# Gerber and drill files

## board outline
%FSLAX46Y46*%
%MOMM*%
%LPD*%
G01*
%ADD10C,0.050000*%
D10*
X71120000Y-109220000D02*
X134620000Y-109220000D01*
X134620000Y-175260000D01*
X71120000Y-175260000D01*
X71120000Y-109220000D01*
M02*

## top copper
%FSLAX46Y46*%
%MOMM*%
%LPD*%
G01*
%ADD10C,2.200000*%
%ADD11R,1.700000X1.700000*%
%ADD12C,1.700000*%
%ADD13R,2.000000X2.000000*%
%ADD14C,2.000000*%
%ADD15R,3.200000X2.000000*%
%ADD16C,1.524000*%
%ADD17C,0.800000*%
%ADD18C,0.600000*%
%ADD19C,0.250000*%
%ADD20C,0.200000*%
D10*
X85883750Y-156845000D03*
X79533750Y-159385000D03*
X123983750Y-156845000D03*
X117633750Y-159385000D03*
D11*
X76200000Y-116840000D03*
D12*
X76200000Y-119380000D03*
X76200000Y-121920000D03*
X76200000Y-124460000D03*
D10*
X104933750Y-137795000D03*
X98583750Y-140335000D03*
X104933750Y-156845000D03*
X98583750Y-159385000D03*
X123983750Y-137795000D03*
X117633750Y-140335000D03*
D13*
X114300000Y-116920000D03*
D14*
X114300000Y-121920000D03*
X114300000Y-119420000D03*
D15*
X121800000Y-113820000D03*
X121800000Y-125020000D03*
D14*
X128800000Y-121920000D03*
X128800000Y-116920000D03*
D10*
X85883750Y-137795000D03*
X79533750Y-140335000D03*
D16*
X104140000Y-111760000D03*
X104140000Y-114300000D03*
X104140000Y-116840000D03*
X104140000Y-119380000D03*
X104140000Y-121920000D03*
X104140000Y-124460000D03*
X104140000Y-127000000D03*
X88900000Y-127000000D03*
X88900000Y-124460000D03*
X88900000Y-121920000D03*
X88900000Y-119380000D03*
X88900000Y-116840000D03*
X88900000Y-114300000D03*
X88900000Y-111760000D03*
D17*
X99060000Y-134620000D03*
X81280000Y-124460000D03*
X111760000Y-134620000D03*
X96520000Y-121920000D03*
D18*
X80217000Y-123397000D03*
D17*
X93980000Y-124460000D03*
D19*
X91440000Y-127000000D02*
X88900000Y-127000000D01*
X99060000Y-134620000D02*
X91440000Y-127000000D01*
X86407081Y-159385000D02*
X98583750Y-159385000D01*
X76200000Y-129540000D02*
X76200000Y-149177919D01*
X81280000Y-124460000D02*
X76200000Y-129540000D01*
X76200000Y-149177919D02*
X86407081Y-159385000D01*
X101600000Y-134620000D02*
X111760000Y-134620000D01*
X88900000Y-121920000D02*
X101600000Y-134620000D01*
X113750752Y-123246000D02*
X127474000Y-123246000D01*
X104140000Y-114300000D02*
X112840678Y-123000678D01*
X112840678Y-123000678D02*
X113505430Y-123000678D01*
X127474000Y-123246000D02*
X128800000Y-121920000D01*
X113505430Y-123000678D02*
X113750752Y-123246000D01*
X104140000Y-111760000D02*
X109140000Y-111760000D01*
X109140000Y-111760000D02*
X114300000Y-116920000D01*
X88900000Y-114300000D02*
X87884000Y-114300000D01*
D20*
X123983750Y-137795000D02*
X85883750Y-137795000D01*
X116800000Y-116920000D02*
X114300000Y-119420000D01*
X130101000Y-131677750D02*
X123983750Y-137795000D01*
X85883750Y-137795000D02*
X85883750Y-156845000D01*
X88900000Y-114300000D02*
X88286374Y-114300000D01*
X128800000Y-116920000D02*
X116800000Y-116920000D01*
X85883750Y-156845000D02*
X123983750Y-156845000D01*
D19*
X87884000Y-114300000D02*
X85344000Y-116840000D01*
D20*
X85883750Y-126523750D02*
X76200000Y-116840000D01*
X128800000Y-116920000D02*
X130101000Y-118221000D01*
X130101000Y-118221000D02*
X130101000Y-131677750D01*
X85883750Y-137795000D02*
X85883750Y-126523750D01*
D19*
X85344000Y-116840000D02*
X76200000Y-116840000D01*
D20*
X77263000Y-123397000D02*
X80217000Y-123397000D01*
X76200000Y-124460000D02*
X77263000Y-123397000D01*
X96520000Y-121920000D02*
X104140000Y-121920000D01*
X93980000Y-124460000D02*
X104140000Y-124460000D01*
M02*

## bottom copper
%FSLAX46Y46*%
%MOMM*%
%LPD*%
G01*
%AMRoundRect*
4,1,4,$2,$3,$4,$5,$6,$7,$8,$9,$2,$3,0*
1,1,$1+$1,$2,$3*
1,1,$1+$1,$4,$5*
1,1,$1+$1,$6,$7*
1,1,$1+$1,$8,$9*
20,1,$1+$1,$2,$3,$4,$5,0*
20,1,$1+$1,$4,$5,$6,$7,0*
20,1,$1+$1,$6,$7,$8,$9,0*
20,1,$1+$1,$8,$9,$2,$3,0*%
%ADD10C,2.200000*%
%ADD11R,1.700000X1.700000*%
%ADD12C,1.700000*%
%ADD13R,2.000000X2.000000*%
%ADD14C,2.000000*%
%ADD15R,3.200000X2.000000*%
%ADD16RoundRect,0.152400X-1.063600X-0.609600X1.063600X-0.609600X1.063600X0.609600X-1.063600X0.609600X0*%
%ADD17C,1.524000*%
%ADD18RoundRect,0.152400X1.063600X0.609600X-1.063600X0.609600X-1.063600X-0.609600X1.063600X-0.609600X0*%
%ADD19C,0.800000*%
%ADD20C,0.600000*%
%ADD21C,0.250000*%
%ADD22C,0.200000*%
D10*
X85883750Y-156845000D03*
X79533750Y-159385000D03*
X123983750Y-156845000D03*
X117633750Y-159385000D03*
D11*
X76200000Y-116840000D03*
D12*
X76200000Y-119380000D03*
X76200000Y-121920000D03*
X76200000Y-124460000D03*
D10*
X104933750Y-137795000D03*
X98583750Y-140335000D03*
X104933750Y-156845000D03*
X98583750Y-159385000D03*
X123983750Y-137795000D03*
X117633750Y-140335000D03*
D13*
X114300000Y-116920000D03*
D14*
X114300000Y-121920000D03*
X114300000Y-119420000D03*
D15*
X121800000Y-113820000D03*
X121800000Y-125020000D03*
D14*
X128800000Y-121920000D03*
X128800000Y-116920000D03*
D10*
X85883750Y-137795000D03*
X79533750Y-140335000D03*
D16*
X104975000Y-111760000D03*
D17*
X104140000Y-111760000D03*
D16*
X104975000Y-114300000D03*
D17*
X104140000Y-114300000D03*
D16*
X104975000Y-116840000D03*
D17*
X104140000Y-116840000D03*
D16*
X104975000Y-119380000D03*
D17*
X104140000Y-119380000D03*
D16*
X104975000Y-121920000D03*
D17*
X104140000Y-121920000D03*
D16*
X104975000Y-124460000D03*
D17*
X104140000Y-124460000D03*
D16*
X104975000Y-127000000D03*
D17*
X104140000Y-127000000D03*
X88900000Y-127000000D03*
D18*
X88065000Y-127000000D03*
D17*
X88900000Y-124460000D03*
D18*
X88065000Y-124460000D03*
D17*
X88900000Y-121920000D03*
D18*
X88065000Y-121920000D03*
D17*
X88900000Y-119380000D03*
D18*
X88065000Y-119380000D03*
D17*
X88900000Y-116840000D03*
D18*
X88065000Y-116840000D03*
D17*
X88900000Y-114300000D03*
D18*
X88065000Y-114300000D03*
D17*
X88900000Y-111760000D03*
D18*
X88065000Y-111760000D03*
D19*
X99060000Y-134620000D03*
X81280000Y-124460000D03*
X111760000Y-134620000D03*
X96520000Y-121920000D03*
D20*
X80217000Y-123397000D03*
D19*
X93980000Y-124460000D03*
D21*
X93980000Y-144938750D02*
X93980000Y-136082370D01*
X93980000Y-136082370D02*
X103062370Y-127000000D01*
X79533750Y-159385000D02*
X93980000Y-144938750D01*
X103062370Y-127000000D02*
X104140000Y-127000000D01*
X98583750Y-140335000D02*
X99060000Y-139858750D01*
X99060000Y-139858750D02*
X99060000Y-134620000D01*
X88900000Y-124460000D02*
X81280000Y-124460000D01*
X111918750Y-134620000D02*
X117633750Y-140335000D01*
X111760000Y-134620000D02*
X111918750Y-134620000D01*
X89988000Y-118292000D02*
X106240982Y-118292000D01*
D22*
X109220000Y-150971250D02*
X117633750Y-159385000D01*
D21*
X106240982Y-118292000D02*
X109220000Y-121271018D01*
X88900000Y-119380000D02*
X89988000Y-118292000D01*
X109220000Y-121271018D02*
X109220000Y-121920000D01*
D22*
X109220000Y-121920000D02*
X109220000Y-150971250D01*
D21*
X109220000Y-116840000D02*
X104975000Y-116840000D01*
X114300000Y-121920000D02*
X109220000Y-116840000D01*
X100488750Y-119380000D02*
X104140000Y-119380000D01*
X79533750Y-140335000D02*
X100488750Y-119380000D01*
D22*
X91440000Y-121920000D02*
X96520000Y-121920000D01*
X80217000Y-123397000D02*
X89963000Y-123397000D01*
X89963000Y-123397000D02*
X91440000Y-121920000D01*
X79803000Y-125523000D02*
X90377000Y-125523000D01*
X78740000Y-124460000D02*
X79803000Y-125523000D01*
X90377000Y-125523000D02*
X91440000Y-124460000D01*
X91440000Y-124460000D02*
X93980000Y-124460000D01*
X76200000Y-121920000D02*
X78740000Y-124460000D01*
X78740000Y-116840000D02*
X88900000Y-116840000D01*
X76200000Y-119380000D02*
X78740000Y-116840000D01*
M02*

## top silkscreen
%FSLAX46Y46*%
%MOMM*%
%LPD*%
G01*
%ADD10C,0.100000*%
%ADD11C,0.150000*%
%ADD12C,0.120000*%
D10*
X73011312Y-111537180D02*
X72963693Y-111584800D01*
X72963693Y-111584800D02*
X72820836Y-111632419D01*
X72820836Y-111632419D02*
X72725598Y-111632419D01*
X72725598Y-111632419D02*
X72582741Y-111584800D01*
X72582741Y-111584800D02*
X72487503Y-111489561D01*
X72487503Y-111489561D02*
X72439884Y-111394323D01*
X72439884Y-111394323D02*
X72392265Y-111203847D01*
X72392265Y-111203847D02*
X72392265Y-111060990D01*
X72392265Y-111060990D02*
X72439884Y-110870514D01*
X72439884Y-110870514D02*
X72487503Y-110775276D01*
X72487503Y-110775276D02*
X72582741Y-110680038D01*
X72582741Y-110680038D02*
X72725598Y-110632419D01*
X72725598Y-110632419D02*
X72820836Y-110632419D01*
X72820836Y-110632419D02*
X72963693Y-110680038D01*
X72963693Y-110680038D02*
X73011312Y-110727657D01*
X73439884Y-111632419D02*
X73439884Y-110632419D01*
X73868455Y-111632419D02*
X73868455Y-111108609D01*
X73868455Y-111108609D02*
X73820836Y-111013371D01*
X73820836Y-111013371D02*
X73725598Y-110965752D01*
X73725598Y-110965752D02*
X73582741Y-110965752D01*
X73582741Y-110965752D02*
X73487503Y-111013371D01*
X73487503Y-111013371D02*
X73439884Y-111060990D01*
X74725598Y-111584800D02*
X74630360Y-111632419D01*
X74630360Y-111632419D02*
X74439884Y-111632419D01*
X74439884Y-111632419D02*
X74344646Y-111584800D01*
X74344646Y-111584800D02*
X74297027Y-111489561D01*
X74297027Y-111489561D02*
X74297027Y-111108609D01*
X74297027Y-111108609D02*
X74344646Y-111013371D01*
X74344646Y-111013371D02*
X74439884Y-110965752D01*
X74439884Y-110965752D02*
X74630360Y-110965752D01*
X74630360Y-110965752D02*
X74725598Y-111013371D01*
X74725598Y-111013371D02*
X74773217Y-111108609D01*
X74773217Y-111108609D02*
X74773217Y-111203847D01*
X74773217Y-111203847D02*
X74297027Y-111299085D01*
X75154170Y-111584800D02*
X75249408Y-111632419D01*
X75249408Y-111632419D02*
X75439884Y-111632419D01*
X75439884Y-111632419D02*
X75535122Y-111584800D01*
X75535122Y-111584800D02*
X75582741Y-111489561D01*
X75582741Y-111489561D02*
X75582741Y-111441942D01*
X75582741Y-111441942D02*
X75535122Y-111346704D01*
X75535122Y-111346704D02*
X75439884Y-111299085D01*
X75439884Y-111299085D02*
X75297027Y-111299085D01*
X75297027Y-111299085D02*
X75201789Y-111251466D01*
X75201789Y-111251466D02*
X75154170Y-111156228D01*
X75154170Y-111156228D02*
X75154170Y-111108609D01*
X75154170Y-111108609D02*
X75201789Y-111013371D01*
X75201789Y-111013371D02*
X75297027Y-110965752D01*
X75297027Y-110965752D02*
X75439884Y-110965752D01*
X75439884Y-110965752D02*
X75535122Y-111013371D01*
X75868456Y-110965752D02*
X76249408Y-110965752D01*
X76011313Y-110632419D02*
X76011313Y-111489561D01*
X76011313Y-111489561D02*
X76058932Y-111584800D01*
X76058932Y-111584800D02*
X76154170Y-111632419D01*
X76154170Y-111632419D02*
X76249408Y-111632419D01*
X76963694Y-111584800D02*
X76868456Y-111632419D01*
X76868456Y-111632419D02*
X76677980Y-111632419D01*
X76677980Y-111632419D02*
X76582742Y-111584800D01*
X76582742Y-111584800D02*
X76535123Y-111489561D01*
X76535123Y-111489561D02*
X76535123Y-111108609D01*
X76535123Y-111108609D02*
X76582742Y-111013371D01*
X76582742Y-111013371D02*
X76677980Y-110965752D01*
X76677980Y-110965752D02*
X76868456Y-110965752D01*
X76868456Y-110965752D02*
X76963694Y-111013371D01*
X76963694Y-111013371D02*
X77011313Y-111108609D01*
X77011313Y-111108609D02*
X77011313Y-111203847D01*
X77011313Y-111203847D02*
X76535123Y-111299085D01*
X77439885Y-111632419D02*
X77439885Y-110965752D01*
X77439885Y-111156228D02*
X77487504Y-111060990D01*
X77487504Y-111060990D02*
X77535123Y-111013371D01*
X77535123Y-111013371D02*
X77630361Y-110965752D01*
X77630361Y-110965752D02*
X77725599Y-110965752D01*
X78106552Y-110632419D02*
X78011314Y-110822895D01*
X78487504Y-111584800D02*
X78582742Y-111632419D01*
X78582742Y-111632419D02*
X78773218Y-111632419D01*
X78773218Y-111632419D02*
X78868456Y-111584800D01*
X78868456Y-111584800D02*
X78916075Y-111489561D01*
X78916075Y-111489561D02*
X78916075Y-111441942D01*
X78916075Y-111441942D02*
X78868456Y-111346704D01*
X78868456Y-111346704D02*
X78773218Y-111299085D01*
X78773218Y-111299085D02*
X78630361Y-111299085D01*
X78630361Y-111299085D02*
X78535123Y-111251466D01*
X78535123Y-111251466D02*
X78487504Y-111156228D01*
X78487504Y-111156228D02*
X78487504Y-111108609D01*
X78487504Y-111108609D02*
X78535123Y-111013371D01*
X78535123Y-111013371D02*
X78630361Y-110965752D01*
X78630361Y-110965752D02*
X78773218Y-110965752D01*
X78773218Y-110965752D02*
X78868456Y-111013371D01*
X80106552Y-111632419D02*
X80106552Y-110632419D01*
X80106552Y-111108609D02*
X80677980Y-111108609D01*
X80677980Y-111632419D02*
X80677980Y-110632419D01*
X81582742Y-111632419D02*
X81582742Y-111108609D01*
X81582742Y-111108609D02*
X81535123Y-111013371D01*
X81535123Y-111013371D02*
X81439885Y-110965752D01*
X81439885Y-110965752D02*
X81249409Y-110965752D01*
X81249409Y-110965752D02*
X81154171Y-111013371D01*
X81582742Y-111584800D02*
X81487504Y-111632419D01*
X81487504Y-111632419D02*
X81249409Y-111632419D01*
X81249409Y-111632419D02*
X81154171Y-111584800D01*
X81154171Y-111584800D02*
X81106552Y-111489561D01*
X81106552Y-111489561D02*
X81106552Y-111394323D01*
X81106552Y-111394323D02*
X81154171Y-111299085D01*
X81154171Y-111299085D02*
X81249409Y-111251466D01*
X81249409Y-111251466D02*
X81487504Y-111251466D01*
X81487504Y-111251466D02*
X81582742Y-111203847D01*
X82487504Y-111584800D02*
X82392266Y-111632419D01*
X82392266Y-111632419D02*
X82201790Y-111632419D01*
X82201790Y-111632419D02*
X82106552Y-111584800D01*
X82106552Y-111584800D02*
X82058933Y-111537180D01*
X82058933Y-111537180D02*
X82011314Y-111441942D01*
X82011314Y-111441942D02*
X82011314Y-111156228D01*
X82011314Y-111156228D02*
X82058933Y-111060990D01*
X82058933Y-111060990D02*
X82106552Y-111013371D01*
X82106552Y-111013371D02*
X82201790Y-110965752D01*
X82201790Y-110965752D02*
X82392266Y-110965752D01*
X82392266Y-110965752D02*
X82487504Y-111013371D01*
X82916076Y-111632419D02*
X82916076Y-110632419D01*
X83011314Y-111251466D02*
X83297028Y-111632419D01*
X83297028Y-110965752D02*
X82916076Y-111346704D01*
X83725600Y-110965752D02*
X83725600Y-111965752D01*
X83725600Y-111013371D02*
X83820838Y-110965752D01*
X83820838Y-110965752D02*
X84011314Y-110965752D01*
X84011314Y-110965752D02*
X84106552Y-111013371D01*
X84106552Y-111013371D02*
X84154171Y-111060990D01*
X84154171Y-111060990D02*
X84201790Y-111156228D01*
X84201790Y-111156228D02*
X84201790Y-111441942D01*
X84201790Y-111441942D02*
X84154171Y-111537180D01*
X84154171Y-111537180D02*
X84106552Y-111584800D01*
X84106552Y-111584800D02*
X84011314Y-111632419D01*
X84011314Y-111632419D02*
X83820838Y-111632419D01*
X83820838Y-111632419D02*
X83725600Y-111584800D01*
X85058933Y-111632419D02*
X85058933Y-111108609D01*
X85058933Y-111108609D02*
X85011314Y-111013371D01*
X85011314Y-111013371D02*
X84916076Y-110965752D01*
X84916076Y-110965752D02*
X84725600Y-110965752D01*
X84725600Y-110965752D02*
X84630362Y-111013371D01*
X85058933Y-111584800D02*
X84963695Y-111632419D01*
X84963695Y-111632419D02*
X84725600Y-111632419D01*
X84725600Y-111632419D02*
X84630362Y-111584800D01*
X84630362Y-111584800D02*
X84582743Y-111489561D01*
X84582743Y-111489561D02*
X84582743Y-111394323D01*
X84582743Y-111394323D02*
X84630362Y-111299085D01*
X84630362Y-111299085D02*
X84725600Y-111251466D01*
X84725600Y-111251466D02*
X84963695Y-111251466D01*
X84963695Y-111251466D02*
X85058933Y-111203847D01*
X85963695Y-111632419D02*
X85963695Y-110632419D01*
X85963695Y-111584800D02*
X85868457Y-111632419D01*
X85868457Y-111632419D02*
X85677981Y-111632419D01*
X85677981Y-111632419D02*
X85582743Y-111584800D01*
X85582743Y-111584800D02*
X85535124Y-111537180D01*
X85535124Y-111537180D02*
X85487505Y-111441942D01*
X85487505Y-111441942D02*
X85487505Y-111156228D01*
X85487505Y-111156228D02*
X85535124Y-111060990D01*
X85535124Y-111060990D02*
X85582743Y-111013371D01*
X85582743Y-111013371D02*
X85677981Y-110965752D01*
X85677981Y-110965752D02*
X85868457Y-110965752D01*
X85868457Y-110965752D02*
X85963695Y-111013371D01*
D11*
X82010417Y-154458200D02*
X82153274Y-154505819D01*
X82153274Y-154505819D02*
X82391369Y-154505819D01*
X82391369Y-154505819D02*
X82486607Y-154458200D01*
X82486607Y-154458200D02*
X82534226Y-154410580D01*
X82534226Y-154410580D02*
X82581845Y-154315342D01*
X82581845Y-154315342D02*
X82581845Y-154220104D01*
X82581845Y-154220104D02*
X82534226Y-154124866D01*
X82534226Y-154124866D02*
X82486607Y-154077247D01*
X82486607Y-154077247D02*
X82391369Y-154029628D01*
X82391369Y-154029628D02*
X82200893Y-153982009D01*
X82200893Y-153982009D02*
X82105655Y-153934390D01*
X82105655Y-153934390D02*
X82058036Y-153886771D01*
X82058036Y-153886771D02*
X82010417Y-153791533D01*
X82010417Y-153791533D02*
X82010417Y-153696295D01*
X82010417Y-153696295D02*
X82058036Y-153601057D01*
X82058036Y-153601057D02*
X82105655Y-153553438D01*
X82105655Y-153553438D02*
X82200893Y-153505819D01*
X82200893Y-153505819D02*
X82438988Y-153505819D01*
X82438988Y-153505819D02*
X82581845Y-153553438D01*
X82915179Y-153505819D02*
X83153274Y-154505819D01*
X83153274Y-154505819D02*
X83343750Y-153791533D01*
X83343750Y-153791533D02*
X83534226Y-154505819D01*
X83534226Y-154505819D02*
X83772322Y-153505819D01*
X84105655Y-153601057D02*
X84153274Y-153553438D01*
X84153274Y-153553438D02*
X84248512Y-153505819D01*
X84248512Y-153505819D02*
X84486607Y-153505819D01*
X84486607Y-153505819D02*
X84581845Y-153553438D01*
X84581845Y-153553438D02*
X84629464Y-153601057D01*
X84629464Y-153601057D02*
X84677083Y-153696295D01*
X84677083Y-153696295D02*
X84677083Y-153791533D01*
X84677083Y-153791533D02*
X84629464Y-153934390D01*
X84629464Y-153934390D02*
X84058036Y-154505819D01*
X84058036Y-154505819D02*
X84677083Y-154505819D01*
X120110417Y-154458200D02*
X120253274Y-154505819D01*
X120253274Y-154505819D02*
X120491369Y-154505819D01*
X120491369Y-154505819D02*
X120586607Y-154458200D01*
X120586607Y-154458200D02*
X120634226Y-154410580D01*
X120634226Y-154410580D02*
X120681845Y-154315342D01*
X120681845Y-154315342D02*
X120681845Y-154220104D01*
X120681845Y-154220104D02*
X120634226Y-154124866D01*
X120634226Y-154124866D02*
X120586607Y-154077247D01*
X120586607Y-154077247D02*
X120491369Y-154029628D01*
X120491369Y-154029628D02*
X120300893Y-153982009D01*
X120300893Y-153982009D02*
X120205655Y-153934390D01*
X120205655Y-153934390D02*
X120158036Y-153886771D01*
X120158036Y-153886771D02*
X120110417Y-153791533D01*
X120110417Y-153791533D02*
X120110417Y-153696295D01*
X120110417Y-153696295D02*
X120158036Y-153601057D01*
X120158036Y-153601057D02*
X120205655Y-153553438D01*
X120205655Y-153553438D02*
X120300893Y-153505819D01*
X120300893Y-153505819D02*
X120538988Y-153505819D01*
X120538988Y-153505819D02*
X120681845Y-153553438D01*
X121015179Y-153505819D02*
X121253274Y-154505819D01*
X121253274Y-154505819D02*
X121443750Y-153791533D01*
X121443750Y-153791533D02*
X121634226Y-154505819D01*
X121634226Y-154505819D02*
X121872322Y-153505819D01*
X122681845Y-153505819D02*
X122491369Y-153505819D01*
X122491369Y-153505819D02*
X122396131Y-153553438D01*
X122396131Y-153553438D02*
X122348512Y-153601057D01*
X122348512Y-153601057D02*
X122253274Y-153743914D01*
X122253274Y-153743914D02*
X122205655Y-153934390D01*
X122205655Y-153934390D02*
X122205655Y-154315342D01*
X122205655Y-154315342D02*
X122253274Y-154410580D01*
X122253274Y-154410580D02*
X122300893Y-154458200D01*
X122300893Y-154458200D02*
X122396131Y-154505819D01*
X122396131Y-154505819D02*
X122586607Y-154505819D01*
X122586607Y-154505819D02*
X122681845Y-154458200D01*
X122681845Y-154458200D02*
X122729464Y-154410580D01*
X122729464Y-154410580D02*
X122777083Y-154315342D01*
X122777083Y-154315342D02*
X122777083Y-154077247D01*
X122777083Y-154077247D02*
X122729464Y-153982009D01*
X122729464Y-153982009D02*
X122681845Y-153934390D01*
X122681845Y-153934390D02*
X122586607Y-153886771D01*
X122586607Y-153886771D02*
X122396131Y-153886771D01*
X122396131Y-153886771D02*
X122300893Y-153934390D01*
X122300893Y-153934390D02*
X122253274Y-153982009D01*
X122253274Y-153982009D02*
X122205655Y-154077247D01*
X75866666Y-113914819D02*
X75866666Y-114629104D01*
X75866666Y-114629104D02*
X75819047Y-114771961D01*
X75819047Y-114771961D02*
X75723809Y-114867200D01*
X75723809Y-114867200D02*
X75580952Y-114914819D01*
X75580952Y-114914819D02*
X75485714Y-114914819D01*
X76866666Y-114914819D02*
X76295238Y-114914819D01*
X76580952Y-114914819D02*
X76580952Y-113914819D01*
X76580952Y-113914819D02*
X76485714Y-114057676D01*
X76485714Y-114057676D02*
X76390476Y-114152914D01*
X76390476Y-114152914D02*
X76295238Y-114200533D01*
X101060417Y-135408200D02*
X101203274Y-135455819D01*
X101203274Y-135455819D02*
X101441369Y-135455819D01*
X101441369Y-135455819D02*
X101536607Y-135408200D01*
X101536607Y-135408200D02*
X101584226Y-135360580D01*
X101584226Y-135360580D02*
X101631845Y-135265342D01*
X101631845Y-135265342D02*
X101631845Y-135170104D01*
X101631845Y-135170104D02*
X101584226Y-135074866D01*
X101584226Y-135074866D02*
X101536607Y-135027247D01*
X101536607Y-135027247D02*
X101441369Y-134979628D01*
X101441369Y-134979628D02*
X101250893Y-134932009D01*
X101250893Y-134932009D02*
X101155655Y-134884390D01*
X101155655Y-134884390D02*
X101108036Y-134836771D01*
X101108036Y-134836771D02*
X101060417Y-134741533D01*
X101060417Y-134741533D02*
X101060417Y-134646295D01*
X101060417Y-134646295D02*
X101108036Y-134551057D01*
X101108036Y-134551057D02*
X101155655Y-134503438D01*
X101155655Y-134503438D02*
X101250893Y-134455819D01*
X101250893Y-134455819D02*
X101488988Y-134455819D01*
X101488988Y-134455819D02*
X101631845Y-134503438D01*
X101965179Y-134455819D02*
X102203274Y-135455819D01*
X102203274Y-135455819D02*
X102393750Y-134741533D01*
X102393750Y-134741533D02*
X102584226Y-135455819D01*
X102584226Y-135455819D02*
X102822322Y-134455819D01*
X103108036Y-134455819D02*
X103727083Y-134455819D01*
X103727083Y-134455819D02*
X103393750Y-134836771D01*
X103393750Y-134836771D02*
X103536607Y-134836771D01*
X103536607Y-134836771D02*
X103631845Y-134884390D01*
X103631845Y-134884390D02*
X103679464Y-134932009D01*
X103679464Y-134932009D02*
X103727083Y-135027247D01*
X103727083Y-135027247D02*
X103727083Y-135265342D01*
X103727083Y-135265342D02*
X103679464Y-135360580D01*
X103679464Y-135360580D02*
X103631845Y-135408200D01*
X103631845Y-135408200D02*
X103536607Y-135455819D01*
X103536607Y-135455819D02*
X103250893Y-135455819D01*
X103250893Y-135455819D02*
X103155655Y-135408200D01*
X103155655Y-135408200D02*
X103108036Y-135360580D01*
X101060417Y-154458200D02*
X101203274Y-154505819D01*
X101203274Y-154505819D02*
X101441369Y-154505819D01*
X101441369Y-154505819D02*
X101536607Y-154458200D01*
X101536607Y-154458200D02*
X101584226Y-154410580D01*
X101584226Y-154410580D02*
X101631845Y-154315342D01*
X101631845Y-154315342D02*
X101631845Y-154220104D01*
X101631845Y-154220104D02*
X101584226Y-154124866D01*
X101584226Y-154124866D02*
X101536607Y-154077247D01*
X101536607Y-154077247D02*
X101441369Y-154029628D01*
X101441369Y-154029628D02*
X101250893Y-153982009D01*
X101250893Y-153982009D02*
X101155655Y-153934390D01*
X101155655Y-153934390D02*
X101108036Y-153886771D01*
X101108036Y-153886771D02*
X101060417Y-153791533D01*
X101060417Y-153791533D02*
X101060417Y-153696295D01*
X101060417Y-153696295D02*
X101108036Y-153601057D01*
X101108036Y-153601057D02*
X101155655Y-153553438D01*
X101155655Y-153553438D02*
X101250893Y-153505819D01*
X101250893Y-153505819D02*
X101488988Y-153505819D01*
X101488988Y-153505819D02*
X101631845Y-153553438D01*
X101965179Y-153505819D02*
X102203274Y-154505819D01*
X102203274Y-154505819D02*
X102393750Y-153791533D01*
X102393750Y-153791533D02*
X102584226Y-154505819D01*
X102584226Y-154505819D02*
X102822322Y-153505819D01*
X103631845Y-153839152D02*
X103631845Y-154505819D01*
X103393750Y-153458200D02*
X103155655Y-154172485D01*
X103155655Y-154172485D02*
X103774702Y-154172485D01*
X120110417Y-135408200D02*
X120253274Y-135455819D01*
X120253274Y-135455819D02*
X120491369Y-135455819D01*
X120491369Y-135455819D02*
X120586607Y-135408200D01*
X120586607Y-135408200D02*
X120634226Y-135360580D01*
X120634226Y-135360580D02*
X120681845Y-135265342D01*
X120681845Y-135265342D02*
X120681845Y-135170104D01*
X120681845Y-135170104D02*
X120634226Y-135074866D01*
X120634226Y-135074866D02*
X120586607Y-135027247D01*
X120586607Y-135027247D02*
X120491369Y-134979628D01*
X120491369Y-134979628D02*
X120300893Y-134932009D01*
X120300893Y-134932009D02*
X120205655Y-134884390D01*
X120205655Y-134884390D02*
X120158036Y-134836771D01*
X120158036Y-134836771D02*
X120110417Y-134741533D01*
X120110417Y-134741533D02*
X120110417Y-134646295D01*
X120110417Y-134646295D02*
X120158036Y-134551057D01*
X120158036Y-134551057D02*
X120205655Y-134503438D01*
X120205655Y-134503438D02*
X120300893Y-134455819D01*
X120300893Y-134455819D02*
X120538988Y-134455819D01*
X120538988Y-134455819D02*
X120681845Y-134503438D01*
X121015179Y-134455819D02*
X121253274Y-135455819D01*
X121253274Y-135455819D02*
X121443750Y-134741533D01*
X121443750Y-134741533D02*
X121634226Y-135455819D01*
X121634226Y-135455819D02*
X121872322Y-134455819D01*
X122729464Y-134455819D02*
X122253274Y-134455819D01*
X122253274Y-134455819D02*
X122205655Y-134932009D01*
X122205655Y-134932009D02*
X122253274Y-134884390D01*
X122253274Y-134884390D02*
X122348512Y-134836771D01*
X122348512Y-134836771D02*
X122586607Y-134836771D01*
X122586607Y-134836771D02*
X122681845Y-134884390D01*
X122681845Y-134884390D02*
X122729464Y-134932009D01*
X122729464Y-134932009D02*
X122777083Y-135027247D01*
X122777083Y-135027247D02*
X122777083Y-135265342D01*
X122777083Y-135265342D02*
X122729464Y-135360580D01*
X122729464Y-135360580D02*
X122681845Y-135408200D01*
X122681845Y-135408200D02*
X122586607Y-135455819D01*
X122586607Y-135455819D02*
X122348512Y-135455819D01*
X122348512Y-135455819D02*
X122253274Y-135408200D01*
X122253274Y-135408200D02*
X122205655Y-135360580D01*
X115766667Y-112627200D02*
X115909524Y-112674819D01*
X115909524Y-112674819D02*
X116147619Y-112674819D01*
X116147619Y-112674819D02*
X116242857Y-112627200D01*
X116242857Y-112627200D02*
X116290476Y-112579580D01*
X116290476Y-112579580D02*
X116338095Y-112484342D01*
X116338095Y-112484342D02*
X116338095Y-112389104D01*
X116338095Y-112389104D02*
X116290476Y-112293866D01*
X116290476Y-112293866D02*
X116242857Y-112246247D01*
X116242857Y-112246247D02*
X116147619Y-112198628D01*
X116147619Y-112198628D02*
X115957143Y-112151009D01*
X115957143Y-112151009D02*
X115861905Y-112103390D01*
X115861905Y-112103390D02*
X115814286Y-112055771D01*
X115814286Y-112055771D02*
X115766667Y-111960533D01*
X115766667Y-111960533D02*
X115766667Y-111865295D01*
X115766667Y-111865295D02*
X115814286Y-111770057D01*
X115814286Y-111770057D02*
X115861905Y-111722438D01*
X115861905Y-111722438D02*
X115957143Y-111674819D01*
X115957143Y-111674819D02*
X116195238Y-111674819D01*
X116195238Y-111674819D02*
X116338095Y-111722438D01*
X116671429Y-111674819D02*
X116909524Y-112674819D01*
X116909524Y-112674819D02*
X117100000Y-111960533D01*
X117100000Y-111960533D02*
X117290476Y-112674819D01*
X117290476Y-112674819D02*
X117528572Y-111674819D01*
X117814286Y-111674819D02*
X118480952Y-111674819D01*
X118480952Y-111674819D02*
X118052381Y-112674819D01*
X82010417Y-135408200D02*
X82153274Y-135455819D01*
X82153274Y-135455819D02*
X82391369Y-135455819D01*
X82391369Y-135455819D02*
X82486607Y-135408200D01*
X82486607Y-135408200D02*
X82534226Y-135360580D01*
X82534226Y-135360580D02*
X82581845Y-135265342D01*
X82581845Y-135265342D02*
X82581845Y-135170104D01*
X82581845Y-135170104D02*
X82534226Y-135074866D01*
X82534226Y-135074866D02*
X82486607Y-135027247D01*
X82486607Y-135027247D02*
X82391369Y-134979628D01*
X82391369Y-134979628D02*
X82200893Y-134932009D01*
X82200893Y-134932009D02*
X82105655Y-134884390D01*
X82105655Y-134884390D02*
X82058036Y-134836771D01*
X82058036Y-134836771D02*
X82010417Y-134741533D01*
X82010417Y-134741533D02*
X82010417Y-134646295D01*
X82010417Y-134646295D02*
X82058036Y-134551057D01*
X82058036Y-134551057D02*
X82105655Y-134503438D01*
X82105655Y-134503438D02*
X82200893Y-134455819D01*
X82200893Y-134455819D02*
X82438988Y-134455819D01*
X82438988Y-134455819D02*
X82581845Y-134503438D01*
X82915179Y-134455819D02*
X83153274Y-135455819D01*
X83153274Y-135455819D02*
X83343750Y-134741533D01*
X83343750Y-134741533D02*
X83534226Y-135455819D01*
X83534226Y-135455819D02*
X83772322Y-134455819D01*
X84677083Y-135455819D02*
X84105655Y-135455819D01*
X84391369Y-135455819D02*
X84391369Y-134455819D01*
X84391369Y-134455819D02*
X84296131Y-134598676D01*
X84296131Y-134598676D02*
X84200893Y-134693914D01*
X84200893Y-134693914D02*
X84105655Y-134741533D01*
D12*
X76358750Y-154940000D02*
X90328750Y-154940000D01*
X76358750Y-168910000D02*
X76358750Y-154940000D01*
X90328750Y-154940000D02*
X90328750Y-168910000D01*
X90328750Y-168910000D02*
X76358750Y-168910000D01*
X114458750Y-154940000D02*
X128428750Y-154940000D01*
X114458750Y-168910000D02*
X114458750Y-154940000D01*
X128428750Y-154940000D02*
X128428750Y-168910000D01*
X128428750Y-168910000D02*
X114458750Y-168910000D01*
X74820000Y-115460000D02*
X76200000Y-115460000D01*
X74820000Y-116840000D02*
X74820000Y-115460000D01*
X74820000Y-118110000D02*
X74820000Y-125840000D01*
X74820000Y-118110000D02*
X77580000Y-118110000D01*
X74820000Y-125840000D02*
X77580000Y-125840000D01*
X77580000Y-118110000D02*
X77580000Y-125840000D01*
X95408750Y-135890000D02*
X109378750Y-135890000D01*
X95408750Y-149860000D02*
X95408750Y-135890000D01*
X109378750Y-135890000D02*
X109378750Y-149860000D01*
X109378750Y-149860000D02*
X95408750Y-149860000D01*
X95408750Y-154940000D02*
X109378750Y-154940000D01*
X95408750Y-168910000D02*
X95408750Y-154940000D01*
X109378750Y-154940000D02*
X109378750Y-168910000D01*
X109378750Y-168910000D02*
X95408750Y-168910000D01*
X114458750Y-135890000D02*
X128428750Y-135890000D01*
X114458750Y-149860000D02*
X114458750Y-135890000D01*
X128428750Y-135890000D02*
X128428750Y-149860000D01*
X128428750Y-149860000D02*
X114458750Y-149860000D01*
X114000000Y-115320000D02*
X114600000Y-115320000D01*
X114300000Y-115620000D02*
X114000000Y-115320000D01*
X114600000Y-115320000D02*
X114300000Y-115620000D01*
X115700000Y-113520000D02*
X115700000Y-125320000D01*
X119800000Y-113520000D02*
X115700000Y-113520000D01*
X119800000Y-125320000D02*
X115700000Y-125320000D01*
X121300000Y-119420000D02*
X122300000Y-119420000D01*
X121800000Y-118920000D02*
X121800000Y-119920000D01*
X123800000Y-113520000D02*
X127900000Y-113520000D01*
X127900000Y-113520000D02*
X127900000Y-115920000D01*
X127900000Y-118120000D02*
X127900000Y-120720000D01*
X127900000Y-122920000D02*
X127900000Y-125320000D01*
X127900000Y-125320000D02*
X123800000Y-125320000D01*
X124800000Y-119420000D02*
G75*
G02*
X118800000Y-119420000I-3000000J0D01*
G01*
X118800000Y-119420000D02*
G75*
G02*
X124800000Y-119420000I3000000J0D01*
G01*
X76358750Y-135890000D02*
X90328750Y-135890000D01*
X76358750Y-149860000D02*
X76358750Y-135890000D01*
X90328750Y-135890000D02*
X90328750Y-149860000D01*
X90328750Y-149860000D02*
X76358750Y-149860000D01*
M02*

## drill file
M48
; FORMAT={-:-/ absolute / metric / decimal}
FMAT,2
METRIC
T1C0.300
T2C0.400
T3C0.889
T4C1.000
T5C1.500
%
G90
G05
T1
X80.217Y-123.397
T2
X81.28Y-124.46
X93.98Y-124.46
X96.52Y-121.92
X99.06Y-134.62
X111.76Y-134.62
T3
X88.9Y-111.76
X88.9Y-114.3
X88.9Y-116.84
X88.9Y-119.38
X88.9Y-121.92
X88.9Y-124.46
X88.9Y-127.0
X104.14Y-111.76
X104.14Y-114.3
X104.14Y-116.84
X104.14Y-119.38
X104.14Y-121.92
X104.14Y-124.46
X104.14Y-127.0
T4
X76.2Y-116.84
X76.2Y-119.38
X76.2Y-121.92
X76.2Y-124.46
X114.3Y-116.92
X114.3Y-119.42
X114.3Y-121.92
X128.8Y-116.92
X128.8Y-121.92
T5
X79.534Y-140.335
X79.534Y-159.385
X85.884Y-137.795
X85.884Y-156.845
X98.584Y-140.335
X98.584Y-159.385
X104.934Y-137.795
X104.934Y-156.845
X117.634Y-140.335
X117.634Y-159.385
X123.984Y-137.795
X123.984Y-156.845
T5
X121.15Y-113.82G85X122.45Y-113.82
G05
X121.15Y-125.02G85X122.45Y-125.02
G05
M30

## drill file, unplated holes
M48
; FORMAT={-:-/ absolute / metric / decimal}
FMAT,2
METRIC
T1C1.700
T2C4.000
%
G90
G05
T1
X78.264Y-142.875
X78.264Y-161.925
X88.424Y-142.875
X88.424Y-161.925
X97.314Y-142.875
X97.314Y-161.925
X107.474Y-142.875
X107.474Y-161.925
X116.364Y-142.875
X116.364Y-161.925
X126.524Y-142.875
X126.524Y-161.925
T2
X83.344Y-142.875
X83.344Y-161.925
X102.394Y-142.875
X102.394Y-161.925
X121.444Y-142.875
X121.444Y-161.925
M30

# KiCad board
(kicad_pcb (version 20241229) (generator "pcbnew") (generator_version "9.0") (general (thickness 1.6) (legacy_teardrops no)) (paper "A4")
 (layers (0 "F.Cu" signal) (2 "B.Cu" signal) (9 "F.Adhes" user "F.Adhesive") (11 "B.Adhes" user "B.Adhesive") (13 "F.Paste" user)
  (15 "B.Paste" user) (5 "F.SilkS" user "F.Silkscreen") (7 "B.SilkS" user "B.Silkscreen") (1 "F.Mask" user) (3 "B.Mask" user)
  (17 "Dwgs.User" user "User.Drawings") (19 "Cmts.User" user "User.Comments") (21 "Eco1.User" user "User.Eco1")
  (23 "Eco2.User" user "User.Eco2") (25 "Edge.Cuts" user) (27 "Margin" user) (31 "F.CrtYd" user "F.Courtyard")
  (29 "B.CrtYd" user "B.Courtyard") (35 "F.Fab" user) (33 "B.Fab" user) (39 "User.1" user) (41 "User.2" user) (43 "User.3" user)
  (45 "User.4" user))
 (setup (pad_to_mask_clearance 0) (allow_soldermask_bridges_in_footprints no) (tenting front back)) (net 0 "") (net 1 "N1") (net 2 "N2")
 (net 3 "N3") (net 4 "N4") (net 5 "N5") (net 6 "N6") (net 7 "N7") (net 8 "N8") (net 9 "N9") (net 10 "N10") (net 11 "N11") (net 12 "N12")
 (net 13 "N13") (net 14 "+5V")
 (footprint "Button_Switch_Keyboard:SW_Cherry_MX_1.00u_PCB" (layer "F.Cu") (at 85.88375 156.845)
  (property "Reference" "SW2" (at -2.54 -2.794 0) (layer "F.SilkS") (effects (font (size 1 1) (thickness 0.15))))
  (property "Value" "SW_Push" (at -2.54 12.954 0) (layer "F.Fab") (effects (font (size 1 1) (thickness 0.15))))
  (fp_line (start -9.525 -1.905) (end 4.445 -1.905) (stroke (width 0.12) (type solid)) (layer "F.SilkS"))
  (fp_line (start -9.525 12.065) (end -9.525 -1.905) (stroke (width 0.12) (type solid)) (layer "F.SilkS"))
  (fp_line (start 4.445 -1.905) (end 4.445 12.065) (stroke (width 0.12) (type solid)) (layer "F.SilkS"))
  (fp_line (start 4.445 12.065) (end -9.525 12.065) (stroke (width 0.12) (type solid)) (layer "F.SilkS"))
  (pad "" np_thru_hole circle (at -7.62 5.08) (size 1.7 1.7) (drill 1.7) (layers "*.Cu" "*.Mask"))
  (pad "" np_thru_hole circle (at -2.54 5.08) (size 4 4) (drill 4) (layers "*.Cu" "*.Mask"))
  (pad "" np_thru_hole circle (at 2.54 5.08) (size 1.7 1.7) (drill 1.7) (layers "*.Cu" "*.Mask"))
  (pad "1" thru_hole circle (at 0 0) (size 2.2 2.2) (drill 1.5) (layers "*.Cu" "*.Mask") (remove_unused_layers no) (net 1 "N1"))
  (pad "2" thru_hole circle (at -6.35 2.54) (size 2.2 2.2) (drill 1.5) (layers "*.Cu" "*.Mask") (remove_unused_layers no) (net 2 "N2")))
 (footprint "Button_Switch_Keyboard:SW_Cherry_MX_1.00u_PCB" (layer "F.Cu") (at 123.98375 156.845)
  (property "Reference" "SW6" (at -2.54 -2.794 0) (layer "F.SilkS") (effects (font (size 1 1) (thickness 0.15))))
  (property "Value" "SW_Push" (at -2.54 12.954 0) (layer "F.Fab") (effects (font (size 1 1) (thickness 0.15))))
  (fp_line (start -9.525 -1.905) (end 4.445 -1.905) (stroke (width 0.12) (type solid)) (layer "F.SilkS"))
  (fp_line (start -9.525 12.065) (end -9.525 -1.905) (stroke (width 0.12) (type solid)) (layer "F.SilkS"))
  (fp_line (start 4.445 -1.905) (end 4.445 12.065) (stroke (width 0.12) (type solid)) (layer "F.SilkS"))
  (fp_line (start 4.445 12.065) (end -9.525 12.065) (stroke (width 0.12) (type solid)) (layer "F.SilkS"))
  (pad "" np_thru_hole circle (at -7.62 5.08) (size 1.7 1.7) (drill 1.7) (layers "*.Cu" "*.Mask"))
  (pad "" np_thru_hole circle (at -2.54 5.08) (size 4 4) (drill 4) (layers "*.Cu" "*.Mask"))
  (pad "" np_thru_hole circle (at 2.54 5.08) (size 1.7 1.7) (drill 1.7) (layers "*.Cu" "*.Mask"))
  (pad "1" thru_hole circle (at 0 0) (size 2.2 2.2) (drill 1.5) (layers "*.Cu" "*.Mask") (remove_unused_layers no) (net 1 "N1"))
  (pad "2" thru_hole circle (at -6.35 2.54) (size 2.2 2.2) (drill 1.5) (layers "*.Cu" "*.Mask") (remove_unused_layers no) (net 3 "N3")))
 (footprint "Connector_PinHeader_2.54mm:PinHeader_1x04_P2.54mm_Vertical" (layer "F.Cu") (at 76.2 116.84)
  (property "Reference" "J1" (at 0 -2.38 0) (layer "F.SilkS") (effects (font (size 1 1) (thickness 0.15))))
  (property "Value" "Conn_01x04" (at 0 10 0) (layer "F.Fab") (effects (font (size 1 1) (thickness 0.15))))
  (fp_line (start -1.38 -1.38) (end 0 -1.38) (stroke (width 0.12) (type solid)) (layer "F.SilkS"))
  (fp_line (start -1.38 0) (end -1.38 -1.38) (stroke (width 0.12) (type solid)) (layer "F.SilkS"))
  (fp_line (start -1.38 1.27) (end -1.38 9) (stroke (width 0.12) (type solid)) (layer "F.SilkS"))
  (fp_line (start -1.38 1.27) (end 1.38 1.27) (stroke (width 0.12) (type solid)) (layer "F.SilkS"))
  (fp_line (start -1.38 9) (end 1.38 9) (stroke (width 0.12) (type solid)) (layer "F.SilkS"))
  (fp_line (start 1.38 1.27) (end 1.38 9) (stroke (width 0.12) (type solid)) (layer "F.SilkS"))
  (pad "1" thru_hole rect (at 0 0) (size 1.7 1.7) (drill 1) (layers "*.Cu" "*.Mask") (remove_unused_layers no) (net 1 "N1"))
  (pad "2" thru_hole circle (at 0 2.54) (size 1.7 1.7) (drill 1) (layers "*.Cu" "*.Mask") (remove_unused_layers no) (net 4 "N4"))
  (pad "3" thru_hole circle (at 0 5.08) (size 1.7 1.7) (drill 1) (layers "*.Cu" "*.Mask") (remove_unused_layers no) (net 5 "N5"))
  (pad "4" thru_hole circle (at 0 7.62) (size 1.7 1.7) (drill 1) (layers "*.Cu" "*.Mask") (remove_unused_layers no) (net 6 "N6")))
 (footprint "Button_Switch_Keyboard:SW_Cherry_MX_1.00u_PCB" (layer "F.Cu") (at 104.93375 137.795)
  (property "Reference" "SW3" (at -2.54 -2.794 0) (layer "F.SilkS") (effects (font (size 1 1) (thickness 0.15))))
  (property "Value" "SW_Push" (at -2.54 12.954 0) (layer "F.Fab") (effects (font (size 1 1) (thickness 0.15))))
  (fp_line (start -9.525 -1.905) (end 4.445 -1.905) (stroke (width 0.12) (type solid)) (layer "F.SilkS"))
  (fp_line (start -9.525 12.065) (end -9.525 -1.905) (stroke (width 0.12) (type solid)) (layer "F.SilkS"))
  (fp_line (start 4.445 -1.905) (end 4.445 12.065) (stroke (width 0.12) (type solid)) (layer "F.SilkS"))
  (fp_line (start 4.445 12.065) (end -9.525 12.065) (stroke (width 0.12) (type solid)) (layer "F.SilkS"))
  (pad "" np_thru_hole circle (at -7.62 5.08) (size 1.7 1.7) (drill 1.7) (layers "*.Cu" "*.Mask"))
  (pad "" np_thru_hole circle (at -2.54 5.08) (size 4 4) (drill 4) (layers "*.Cu" "*.Mask"))
  (pad "" np_thru_hole circle (at 2.54 5.08) (size 1.7 1.7) (drill 1.7) (layers "*.Cu" "*.Mask"))
  (pad "1" thru_hole circle (at 0 0) (size 2.2 2.2) (drill 1.5) (layers "*.Cu" "*.Mask") (remove_unused_layers no) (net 1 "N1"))
  (pad "2" thru_hole circle (at -6.35 2.54) (size 2.2 2.2) (drill 1.5) (layers "*.Cu" "*.Mask") (remove_unused_layers no) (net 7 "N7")))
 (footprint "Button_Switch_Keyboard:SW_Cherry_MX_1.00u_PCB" (layer "F.Cu") (at 104.93375 156.845)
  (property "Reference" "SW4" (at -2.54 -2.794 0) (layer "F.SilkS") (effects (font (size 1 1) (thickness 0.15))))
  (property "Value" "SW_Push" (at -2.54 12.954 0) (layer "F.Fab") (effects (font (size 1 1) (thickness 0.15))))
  (fp_line (start -9.525 -1.905) (end 4.445 -1.905) (stroke (width 0.12) (type solid)) (layer "F.SilkS"))
  (fp_line (start -9.525 12.065) (end -9.525 -1.905) (stroke (width 0.12) (type solid)) (layer "F.SilkS"))
  (fp_line (start 4.445 -1.905) (end 4.445 12.065) (stroke (width 0.12) (type solid)) (layer "F.SilkS"))
  (fp_line (start 4.445 12.065) (end -9.525 12.065) (stroke (width 0.12) (type solid)) (layer "F.SilkS"))
  (pad "" np_thru_hole circle (at -7.62 5.08) (size 1.7 1.7) (drill 1.7) (layers "*.Cu" "*.Mask"))
  (pad "" np_thru_hole circle (at -2.54 5.08) (size 4 4) (drill 4) (layers "*.Cu" "*.Mask"))
  (pad "" np_thru_hole circle (at 2.54 5.08) (size 1.7 1.7) (drill 1.7) (layers "*.Cu" "*.Mask"))
  (pad "1" thru_hole circle (at 0 0) (size 2.2 2.2) (drill 1.5) (layers "*.Cu" "*.Mask") (remove_unused_layers no) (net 1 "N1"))
  (pad "2" thru_hole circle (at -6.35 2.54) (size 2.2 2.2) (drill 1.5) (layers "*.Cu" "*.Mask") (remove_unused_layers no) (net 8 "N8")))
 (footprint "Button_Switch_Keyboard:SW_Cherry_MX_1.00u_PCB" (layer "F.Cu") (at 123.98375 137.795)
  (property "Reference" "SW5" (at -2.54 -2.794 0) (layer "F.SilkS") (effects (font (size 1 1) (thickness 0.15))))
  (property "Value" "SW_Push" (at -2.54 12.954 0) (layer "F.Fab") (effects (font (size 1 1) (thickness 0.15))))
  (fp_line (start -9.525 -1.905) (end 4.445 -1.905) (stroke (width 0.12) (type solid)) (layer "F.SilkS"))
  (fp_line (start -9.525 12.065) (end -9.525 -1.905) (stroke (width 0.12) (type solid)) (layer "F.SilkS"))
  (fp_line (start 4.445 -1.905) (end 4.445 12.065) (stroke (width 0.12) (type solid)) (layer "F.SilkS"))
  (fp_line (start 4.445 12.065) (end -9.525 12.065) (stroke (width 0.12) (type solid)) (layer "F.SilkS"))
  (pad "" np_thru_hole circle (at -7.62 5.08) (size 1.7 1.7) (drill 1.7) (layers "*.Cu" "*.Mask"))
  (pad "" np_thru_hole circle (at -2.54 5.08) (size 4 4) (drill 4) (layers "*.Cu" "*.Mask"))
  (pad "" np_thru_hole circle (at 2.54 5.08) (size 1.7 1.7) (drill 1.7) (layers "*.Cu" "*.Mask"))
  (pad "1" thru_hole circle (at 0 0) (size 2.2 2.2) (drill 1.5) (layers "*.Cu" "*.Mask") (remove_unused_layers no) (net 1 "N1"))
  (pad "2" thru_hole circle (at -6.35 2.54) (size 2.2 2.2) (drill 1.5) (layers "*.Cu" "*.Mask") (remove_unused_layers no) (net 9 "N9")))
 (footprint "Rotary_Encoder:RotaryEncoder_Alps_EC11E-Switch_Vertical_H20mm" (layer "F.Cu") (at 114.3 116.92)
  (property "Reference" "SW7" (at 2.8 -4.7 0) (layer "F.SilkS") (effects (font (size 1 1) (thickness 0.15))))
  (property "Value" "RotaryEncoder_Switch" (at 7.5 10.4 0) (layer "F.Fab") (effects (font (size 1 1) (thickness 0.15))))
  (fp_line (start -0.3 -1.6) (end 0.3 -1.6) (stroke (width 0.12) (type solid)) (layer "F.SilkS"))
  (fp_line (start 0 -1.3) (end -0.3 -1.6) (stroke (width 0.12) (type solid)) (layer "F.SilkS"))
  (fp_line (start 0.3 -1.6) (end 0 -1.3) (stroke (width 0.12) (type solid)) (layer "F.SilkS"))
  (fp_line (start 1.4 -3.4) (end 1.4 8.4) (stroke (width 0.12) (type solid)) (layer "F.SilkS"))
  (fp_line (start 5.5 -3.4) (end 1.4 -3.4) (stroke (width 0.12) (type solid)) (layer "F.SilkS"))
  (fp_line (start 5.5 8.4) (end 1.4 8.4) (stroke (width 0.12) (type solid)) (layer "F.SilkS"))
  (fp_line (start 7 2.5) (end 8 2.5) (stroke (width 0.12) (type solid)) (layer "F.SilkS"))
  (fp_line (start 7.5 2) (end 7.5 3) (stroke (width 0.12) (type solid)) (layer "F.SilkS"))
  (fp_line (start 9.5 -3.4) (end 13.6 -3.4) (stroke (width 0.12) (type solid)) (layer "F.SilkS"))
  (fp_line (start 13.6 -3.4) (end 13.6 -1) (stroke (width 0.12) (type solid)) (layer "F.SilkS"))
  (fp_line (start 13.6 1.2) (end 13.6 3.8) (stroke (width 0.12) (type solid)) (layer "F.SilkS"))
  (fp_line (start 13.6 6) (end 13.6 8.4) (stroke (width 0.12) (type solid)) (layer "F.SilkS"))
  (fp_line (start 13.6 8.4) (end 9.5 8.4) (stroke (width 0.12) (type solid)) (layer "F.SilkS"))
  (fp_circle (center 7.5 2.5) (end 10.5 2.5) (stroke (width 0.12) (type solid)) (fill no) (layer "F.SilkS"))
  (pad "A" thru_hole rect (at 0 0) (size 2 2) (drill 1) (layers "*.Cu" "*.Mask") (remove_unused_layers no) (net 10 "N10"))
  (pad "B" thru_hole circle (at 0 5) (size 2 2) (drill 1) (layers "*.Cu" "*.Mask") (remove_unused_layers no) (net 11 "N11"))
  (pad "C" thru_hole circle (at 0 2.5) (size 2 2) (drill 1) (layers "*.Cu" "*.Mask") (remove_unused_layers no) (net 1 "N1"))
  (pad "MP" thru_hole rect (at 7.5 -3.1) (size 3.2 2) (drill oval 2.8 1.5) (layers "*.Cu" "*.Mask") (remove_unused_layers no))
  (pad "MP" thru_hole rect (at 7.5 8.1) (size 3.2 2) (drill oval 2.8 1.5) (layers "*.Cu" "*.Mask") (remove_unused_layers no))
  (pad "S1" thru_hole circle (at 14.5 5) (size 2 2) (drill 1) (layers "*.Cu" "*.Mask") (remove_unused_layers no) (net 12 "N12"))
  (pad "S2" thru_hole circle (at 14.5 0) (size 2 2) (drill 1) (layers "*.Cu" "*.Mask") (remove_unused_layers no) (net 1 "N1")))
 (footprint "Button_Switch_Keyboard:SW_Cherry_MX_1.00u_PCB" (layer "F.Cu") (at 85.88375 137.795)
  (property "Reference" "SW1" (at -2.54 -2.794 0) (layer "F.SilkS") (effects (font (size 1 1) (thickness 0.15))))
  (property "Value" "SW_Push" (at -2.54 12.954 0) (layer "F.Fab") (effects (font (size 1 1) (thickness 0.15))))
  (fp_line (start -9.525 -1.905) (end 4.445 -1.905) (stroke (width 0.12) (type solid)) (layer "F.SilkS"))
  (fp_line (start -9.525 12.065) (end -9.525 -1.905) (stroke (width 0.12) (type solid)) (layer "F.SilkS"))
  (fp_line (start 4.445 -1.905) (end 4.445 12.065) (stroke (width 0.12) (type solid)) (layer "F.SilkS"))
  (fp_line (start 4.445 12.065) (end -9.525 12.065) (stroke (width 0.12) (type solid)) (layer "F.SilkS"))
  (pad "" np_thru_hole circle (at -7.62 5.08) (size 1.7 1.7) (drill 1.7) (layers "*.Cu" "*.Mask"))
  (pad "" np_thru_hole circle (at -2.54 5.08) (size 4 4) (drill 4) (layers "*.Cu" "*.Mask"))
  (pad "" np_thru_hole circle (at 2.54 5.08) (size 1.7 1.7) (drill 1.7) (layers "*.Cu" "*.Mask"))
  (pad "1" thru_hole circle (at 0 0) (size 2.2 2.2) (drill 1.5) (layers "*.Cu" "*.Mask") (remove_unused_layers no) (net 1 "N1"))
  (pad "2" thru_hole circle (at -6.35 2.54) (size 2.2 2.2) (drill 1.5) (layers "*.Cu" "*.Mask") (remove_unused_layers no) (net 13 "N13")))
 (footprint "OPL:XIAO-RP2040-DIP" (layer "B.Cu") (at 96.52 119.38 180)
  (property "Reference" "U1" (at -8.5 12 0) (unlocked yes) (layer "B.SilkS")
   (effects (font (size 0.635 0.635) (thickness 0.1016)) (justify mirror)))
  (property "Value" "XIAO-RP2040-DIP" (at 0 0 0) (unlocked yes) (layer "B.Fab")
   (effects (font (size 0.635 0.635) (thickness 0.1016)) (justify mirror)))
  (pad "1" smd roundrect (at -8.455 7.62) (size 2.432 1.524) (layers "B.Cu" "B.Mask") (roundrect_rratio 0.1) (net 10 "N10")
   (thermal_bridge_angle 45))
  (pad "1" thru_hole circle (at -7.62 7.62) (size 1.524 1.524) (drill 0.889) (layers "*.Cu" "*.Mask") (remove_unused_layers no)
   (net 10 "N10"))
  (pad "2" smd roundrect (at -8.455 5.08) (size 2.432 1.524) (layers "B.Cu" "B.Mask") (roundrect_rratio 0.1) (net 12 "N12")
   (thermal_bridge_angle 45))
  (pad "2" thru_hole circle (at -7.62 5.08) (size 1.524 1.524) (drill 0.889) (layers "*.Cu" "*.Mask") (remove_unused_layers no)
   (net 12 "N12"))
  (pad "3" smd roundrect (at -8.455 2.54) (size 2.432 1.524) (layers "B.Cu" "B.Mask") (roundrect_rratio 0.1) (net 11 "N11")
   (thermal_bridge_angle 45))
  (pad "3" thru_hole circle (at -7.62 2.54) (size 1.524 1.524) (drill 0.889) (layers "*.Cu" "*.Mask") (remove_unused_layers no)
   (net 11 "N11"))
  (pad "4" smd roundrect (at -8.455 0) (size 2.432 1.524) (layers "B.Cu" "B.Mask") (roundrect_rratio 0.1) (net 13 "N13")
   (thermal_bridge_angle 45))
  (pad "4" thru_hole circle (at -7.62 0) (size 1.524 1.524) (drill 0.889) (layers "*.Cu" "*.Mask") (remove_unused_layers no) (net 13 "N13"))
  (pad "5" smd roundrect (at -8.455 -2.54) (size 2.432 1.524) (layers "B.Cu" "B.Mask") (roundrect_rratio 0.1) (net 6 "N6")
   (thermal_bridge_angle 45))
  (pad "5" thru_hole circle (at -7.62 -2.54) (size 1.524 1.524) (drill 0.889) (layers "*.Cu" "*.Mask") (remove_unused_layers no)
   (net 6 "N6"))
  (pad "6" smd roundrect (at -8.455 -5.08) (size 2.432 1.524) (layers "B.Cu" "B.Mask") (roundrect_rratio 0.1) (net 5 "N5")
   (thermal_bridge_angle 45))
  (pad "6" thru_hole circle (at -7.62 -5.08) (size 1.524 1.524) (drill 0.889) (layers "*.Cu" "*.Mask") (remove_unused_layers no)
   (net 5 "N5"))
  (pad "7" smd roundrect (at -8.455 -7.62) (size 2.432 1.524) (layers "B.Cu" "B.Mask") (roundrect_rratio 0.1) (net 2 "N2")
   (thermal_bridge_angle 45))
  (pad "7" thru_hole circle (at -7.62 -7.62) (size 1.524 1.524) (drill 0.889) (layers "*.Cu" "*.Mask") (remove_unused_layers no)
   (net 2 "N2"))
  (pad "8" thru_hole circle (at 7.62 -7.62 180) (size 1.524 1.524) (drill 0.889) (layers "*.Cu" "*.Mask") (remove_unused_layers no)
   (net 7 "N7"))
  (pad "8" smd roundrect (at 8.455 -7.62 180) (size 2.432 1.524) (layers "B.Cu" "B.Mask") (roundrect_rratio 0.1) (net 7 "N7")
   (thermal_bridge_angle 45))
  (pad "9" thru_hole circle (at 7.62 -5.08 180) (size 1.524 1.524) (drill 0.889) (layers "*.Cu" "*.Mask") (remove_unused_layers no)
   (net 8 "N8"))
  (pad "9" smd roundrect (at 8.455 -5.08 180) (size 2.432 1.524) (layers "B.Cu" "B.Mask") (roundrect_rratio 0.1) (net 8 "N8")
   (thermal_bridge_angle 45))
  (pad "10" thru_hole circle (at 7.62 -2.54 180) (size 1.524 1.524) (drill 0.889) (layers "*.Cu" "*.Mask") (remove_unused_layers no)
   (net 9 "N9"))
  (pad "10" smd roundrect (at 8.455 -2.54 180) (size 2.432 1.524) (layers "B.Cu" "B.Mask") (roundrect_rratio 0.1) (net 9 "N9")
   (thermal_bridge_angle 45))
  (pad "11" thru_hole circle (at 7.62 0 180) (size 1.524 1.524) (drill 0.889) (layers "*.Cu" "*.Mask") (remove_unused_layers no)
   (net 3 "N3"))
  (pad "11" smd roundrect (at 8.455 0 180) (size 2.432 1.524) (layers "B.Cu" "B.Mask") (roundrect_rratio 0.1) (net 3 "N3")
   (thermal_bridge_angle 45))
  (pad "12" thru_hole circle (at 7.62 2.54 180) (size 1.524 1.524) (drill 0.889) (layers "*.Cu" "*.Mask") (remove_unused_layers no)
   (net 4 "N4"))
  (pad "12" smd roundrect (at 8.455 2.54 180) (size 2.432 1.524) (layers "B.Cu" "B.Mask") (roundrect_rratio 0.1) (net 4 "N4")
   (thermal_bridge_angle 45))
  (pad "13" thru_hole circle (at 7.62 5.08 180) (size 1.524 1.524) (drill 0.889) (layers "*.Cu" "*.Mask") (remove_unused_layers no)
   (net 1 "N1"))
  (pad "13" smd roundrect (at 8.455 5.08 180) (size 2.432 1.524) (layers "B.Cu" "B.Mask") (roundrect_rratio 0.1) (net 1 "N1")
   (thermal_bridge_angle 45))
  (pad "14" thru_hole circle (at 7.62 7.62 180) (size 1.524 1.524) (drill 0.889) (layers "*.Cu" "*.Mask") (remove_unused_layers no)
   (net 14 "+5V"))
  (pad "14" smd roundrect (at 8.455 7.62 180) (size 2.432 1.524) (layers "B.Cu" "B.Mask") (roundrect_rratio 0.1) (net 14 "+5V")
   (thermal_bridge_angle 45)))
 (gr_rect (start 71.12 109.22) (end 134.62 175.26) (stroke (width 0.05) (type default)) (fill no) (layer "Edge.Cuts"))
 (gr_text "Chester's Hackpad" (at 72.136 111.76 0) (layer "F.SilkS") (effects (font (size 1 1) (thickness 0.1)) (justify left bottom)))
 (segment (start 93.98 144.93875) (end 93.98 136.08237) (width 0.25) (layer "B.Cu") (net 2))
 (segment (start 93.98 136.08237) (end 103.06237 127) (width 0.25) (layer "B.Cu") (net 2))
 (segment (start 79.53375 159.385) (end 93.98 144.93875) (width 0.25) (layer "B.Cu") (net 2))
 (segment (start 103.06237 127) (end 104.14 127) (width 0.25) (layer "B.Cu") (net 2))
 (segment (start 91.44 127) (end 88.9 127) (width 0.25) (layer "F.Cu") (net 7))
 (segment (start 99.06 134.62) (end 91.44 127) (width 0.25) (layer "F.Cu") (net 7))
 (via (at 99.06 134.62) (size 0.8) (drill 0.4) (layers "F.Cu" "B.Cu") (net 7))
 (segment (start 98.58375 140.335) (end 99.06 139.85875) (width 0.25) (layer "B.Cu") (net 7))
 (segment (start 99.06 139.85875) (end 99.06 134.62) (width 0.25) (layer "B.Cu") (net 7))
 (segment (start 86.407081 159.385) (end 98.58375 159.385) (width 0.25) (layer "F.Cu") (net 8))
 (segment (start 76.2 129.54) (end 76.2 149.177919) (width 0.25) (layer "F.Cu") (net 8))
 (segment (start 81.28 124.46) (end 76.2 129.54) (width 0.25) (layer "F.Cu") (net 8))
 (segment (start 76.2 149.177919) (end 86.407081 159.385) (width 0.25) (layer "F.Cu") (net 8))
 (via (at 81.28 124.46) (size 0.8) (drill 0.4) (layers "F.Cu" "B.Cu") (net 8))
 (segment (start 88.9 124.46) (end 81.28 124.46) (width 0.25) (layer "B.Cu") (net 8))
 (segment (start 101.6 134.62) (end 111.76 134.62) (width 0.25) (layer "F.Cu") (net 9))
 (segment (start 88.9 121.92) (end 101.6 134.62) (width 0.25) (layer "F.Cu") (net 9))
 (via (at 111.76 134.62) (size 0.8) (drill 0.4) (layers "F.Cu" "B.Cu") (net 9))
 (segment (start 111.91875 134.62) (end 117.63375 140.335) (width 0.25) (layer "B.Cu") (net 9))
 (segment (start 111.76 134.62) (end 111.91875 134.62) (width 0.25) (layer "B.Cu") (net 9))
 (segment (start 89.988 118.292) (end 106.240982 118.292) (width 0.25) (layer "B.Cu") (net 3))
 (segment (start 109.22 150.97125) (end 117.63375 159.385) (width 0.2) (layer "B.Cu") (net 3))
 (segment (start 106.240982 118.292) (end 109.22 121.271018) (width 0.25) (layer "B.Cu") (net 3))
 (segment (start 88.9 119.38) (end 89.988 118.292) (width 0.25) (layer "B.Cu") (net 3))
 (segment (start 109.22 121.271018) (end 109.22 121.92) (width 0.25) (layer "B.Cu") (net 3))
 (segment (start 109.22 121.92) (end 109.22 150.97125) (width 0.2) (layer "B.Cu") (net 3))
 (segment (start 113.750752 123.246) (end 127.474 123.246) (width 0.25) (layer "F.Cu") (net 12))
 (segment (start 104.14 114.3) (end 112.840678 123.000678) (width 0.25) (layer "F.Cu") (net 12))
 (segment (start 112.840678 123.000678) (end 113.50543 123.000678) (width 0.25) (layer "F.Cu") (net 12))
 (segment (start 127.474 123.246) (end 128.8 121.92) (width 0.25) (layer "F.Cu") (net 12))
 (segment (start 113.50543 123.000678) (end 113.750752 123.246) (width 0.25) (layer "F.Cu") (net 12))
 (segment (start 104.14 111.76) (end 109.14 111.76) (width 0.25) (layer "F.Cu") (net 10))
 (segment (start 109.14 111.76) (end 114.3 116.92) (width 0.25) (layer "F.Cu") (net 10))
 (segment (start 109.22 116.84) (end 104.975 116.84) (width 0.25) (layer "B.Cu") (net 11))
 (segment (start 114.3 121.92) (end 109.22 116.84) (width 0.25) (layer "B.Cu") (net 11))
 (segment (start 100.48875 119.38) (end 104.14 119.38) (width 0.25) (layer "B.Cu") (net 13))
 (segment (start 79.53375 140.335) (end 100.48875 119.38) (width 0.25) (layer "B.Cu") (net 13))
 (segment (start 88.9 114.3) (end 87.884 114.3) (width 0.25) (layer "F.Cu") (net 1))
 (segment (start 123.98375 137.795) (end 85.88375 137.795) (width 0.2) (layer "F.Cu") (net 1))
 (segment (start 116.8 116.92) (end 114.3 119.42) (width 0.2) (layer "F.Cu") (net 1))
 (segment (start 130.101 131.67775) (end 123.98375 137.795) (width 0.2) (layer "F.Cu") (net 1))
 (segment (start 85.88375 137.795) (end 85.88375 156.845) (width 0.2) (layer "F.Cu") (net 1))
 (segment (start 88.9 114.3) (end 88.286374 114.3) (width 0.2) (layer "F.Cu") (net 1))
 (segment (start 128.8 116.92) (end 116.8 116.92) (width 0.2) (layer "F.Cu") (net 1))
 (segment (start 85.88375 156.845) (end 123.98375 156.845) (width 0.2) (layer "F.Cu") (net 1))
 (segment (start 87.884 114.3) (end 85.344 116.84) (width 0.25) (layer "F.Cu") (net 1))
 (segment (start 85.88375 126.52375) (end 76.2 116.84) (width 0.2) (layer "F.Cu") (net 1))
 (segment (start 128.8 116.92) (end 130.101 118.221) (width 0.2) (layer "F.Cu") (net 1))
 (segment (start 130.101 118.221) (end 130.101 131.67775) (width 0.2) (layer "F.Cu") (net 1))
 (segment (start 85.88375 137.795) (end 85.88375 126.52375) (width 0.2) (layer "F.Cu") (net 1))
 (segment (start 85.344 116.84) (end 76.2 116.84) (width 0.25) (layer "F.Cu") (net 1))
 (segment (start 77.263 123.397) (end 80.217 123.397) (width 0.2) (layer "F.Cu") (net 6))
 (segment (start 76.2 124.46) (end 77.263 123.397) (width 0.2) (layer "F.Cu") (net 6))
 (segment (start 96.52 121.92) (end 104.14 121.92) (width 0.2) (layer "F.Cu") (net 6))
 (via (at 96.52 121.92) (size 0.8) (drill 0.4) (layers "F.Cu" "B.Cu") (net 6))
 (via (at 80.217 123.397) (size 0.6) (drill 0.3) (layers "F.Cu" "B.Cu") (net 6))
 (segment (start 91.44 121.92) (end 96.52 121.92) (width 0.2) (layer "B.Cu") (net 6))
 (segment (start 80.217 123.397) (end 89.963 123.397) (width 0.2) (layer "B.Cu") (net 6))
 (segment (start 89.963 123.397) (end 91.44 121.92) (width 0.2) (layer "B.Cu") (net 6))
 (segment (start 93.98 124.46) (end 104.14 124.46) (width 0.2) (layer "F.Cu") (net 5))
 (via (at 93.98 124.46) (size 0.8) (drill 0.4) (layers "F.Cu" "B.Cu") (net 5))
 (segment (start 79.803 125.523) (end 90.377 125.523) (width 0.2) (layer "B.Cu") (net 5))
 (segment (start 78.74 124.46) (end 79.803 125.523) (width 0.2) (layer "B.Cu") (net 5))
 (segment (start 90.377 125.523) (end 91.44 124.46) (width 0.2) (layer "B.Cu") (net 5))
 (segment (start 91.44 124.46) (end 93.98 124.46) (width 0.2) (layer "B.Cu") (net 5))
 (segment (start 76.2 121.92) (end 78.74 124.46) (width 0.2) (layer "B.Cu") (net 5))
 (segment (start 78.74 116.84) (end 88.9 116.84) (width 0.2) (layer "B.Cu") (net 4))
 (segment (start 76.2 119.38) (end 78.74 116.84) (width 0.2) (layer "B.Cu") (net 4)))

